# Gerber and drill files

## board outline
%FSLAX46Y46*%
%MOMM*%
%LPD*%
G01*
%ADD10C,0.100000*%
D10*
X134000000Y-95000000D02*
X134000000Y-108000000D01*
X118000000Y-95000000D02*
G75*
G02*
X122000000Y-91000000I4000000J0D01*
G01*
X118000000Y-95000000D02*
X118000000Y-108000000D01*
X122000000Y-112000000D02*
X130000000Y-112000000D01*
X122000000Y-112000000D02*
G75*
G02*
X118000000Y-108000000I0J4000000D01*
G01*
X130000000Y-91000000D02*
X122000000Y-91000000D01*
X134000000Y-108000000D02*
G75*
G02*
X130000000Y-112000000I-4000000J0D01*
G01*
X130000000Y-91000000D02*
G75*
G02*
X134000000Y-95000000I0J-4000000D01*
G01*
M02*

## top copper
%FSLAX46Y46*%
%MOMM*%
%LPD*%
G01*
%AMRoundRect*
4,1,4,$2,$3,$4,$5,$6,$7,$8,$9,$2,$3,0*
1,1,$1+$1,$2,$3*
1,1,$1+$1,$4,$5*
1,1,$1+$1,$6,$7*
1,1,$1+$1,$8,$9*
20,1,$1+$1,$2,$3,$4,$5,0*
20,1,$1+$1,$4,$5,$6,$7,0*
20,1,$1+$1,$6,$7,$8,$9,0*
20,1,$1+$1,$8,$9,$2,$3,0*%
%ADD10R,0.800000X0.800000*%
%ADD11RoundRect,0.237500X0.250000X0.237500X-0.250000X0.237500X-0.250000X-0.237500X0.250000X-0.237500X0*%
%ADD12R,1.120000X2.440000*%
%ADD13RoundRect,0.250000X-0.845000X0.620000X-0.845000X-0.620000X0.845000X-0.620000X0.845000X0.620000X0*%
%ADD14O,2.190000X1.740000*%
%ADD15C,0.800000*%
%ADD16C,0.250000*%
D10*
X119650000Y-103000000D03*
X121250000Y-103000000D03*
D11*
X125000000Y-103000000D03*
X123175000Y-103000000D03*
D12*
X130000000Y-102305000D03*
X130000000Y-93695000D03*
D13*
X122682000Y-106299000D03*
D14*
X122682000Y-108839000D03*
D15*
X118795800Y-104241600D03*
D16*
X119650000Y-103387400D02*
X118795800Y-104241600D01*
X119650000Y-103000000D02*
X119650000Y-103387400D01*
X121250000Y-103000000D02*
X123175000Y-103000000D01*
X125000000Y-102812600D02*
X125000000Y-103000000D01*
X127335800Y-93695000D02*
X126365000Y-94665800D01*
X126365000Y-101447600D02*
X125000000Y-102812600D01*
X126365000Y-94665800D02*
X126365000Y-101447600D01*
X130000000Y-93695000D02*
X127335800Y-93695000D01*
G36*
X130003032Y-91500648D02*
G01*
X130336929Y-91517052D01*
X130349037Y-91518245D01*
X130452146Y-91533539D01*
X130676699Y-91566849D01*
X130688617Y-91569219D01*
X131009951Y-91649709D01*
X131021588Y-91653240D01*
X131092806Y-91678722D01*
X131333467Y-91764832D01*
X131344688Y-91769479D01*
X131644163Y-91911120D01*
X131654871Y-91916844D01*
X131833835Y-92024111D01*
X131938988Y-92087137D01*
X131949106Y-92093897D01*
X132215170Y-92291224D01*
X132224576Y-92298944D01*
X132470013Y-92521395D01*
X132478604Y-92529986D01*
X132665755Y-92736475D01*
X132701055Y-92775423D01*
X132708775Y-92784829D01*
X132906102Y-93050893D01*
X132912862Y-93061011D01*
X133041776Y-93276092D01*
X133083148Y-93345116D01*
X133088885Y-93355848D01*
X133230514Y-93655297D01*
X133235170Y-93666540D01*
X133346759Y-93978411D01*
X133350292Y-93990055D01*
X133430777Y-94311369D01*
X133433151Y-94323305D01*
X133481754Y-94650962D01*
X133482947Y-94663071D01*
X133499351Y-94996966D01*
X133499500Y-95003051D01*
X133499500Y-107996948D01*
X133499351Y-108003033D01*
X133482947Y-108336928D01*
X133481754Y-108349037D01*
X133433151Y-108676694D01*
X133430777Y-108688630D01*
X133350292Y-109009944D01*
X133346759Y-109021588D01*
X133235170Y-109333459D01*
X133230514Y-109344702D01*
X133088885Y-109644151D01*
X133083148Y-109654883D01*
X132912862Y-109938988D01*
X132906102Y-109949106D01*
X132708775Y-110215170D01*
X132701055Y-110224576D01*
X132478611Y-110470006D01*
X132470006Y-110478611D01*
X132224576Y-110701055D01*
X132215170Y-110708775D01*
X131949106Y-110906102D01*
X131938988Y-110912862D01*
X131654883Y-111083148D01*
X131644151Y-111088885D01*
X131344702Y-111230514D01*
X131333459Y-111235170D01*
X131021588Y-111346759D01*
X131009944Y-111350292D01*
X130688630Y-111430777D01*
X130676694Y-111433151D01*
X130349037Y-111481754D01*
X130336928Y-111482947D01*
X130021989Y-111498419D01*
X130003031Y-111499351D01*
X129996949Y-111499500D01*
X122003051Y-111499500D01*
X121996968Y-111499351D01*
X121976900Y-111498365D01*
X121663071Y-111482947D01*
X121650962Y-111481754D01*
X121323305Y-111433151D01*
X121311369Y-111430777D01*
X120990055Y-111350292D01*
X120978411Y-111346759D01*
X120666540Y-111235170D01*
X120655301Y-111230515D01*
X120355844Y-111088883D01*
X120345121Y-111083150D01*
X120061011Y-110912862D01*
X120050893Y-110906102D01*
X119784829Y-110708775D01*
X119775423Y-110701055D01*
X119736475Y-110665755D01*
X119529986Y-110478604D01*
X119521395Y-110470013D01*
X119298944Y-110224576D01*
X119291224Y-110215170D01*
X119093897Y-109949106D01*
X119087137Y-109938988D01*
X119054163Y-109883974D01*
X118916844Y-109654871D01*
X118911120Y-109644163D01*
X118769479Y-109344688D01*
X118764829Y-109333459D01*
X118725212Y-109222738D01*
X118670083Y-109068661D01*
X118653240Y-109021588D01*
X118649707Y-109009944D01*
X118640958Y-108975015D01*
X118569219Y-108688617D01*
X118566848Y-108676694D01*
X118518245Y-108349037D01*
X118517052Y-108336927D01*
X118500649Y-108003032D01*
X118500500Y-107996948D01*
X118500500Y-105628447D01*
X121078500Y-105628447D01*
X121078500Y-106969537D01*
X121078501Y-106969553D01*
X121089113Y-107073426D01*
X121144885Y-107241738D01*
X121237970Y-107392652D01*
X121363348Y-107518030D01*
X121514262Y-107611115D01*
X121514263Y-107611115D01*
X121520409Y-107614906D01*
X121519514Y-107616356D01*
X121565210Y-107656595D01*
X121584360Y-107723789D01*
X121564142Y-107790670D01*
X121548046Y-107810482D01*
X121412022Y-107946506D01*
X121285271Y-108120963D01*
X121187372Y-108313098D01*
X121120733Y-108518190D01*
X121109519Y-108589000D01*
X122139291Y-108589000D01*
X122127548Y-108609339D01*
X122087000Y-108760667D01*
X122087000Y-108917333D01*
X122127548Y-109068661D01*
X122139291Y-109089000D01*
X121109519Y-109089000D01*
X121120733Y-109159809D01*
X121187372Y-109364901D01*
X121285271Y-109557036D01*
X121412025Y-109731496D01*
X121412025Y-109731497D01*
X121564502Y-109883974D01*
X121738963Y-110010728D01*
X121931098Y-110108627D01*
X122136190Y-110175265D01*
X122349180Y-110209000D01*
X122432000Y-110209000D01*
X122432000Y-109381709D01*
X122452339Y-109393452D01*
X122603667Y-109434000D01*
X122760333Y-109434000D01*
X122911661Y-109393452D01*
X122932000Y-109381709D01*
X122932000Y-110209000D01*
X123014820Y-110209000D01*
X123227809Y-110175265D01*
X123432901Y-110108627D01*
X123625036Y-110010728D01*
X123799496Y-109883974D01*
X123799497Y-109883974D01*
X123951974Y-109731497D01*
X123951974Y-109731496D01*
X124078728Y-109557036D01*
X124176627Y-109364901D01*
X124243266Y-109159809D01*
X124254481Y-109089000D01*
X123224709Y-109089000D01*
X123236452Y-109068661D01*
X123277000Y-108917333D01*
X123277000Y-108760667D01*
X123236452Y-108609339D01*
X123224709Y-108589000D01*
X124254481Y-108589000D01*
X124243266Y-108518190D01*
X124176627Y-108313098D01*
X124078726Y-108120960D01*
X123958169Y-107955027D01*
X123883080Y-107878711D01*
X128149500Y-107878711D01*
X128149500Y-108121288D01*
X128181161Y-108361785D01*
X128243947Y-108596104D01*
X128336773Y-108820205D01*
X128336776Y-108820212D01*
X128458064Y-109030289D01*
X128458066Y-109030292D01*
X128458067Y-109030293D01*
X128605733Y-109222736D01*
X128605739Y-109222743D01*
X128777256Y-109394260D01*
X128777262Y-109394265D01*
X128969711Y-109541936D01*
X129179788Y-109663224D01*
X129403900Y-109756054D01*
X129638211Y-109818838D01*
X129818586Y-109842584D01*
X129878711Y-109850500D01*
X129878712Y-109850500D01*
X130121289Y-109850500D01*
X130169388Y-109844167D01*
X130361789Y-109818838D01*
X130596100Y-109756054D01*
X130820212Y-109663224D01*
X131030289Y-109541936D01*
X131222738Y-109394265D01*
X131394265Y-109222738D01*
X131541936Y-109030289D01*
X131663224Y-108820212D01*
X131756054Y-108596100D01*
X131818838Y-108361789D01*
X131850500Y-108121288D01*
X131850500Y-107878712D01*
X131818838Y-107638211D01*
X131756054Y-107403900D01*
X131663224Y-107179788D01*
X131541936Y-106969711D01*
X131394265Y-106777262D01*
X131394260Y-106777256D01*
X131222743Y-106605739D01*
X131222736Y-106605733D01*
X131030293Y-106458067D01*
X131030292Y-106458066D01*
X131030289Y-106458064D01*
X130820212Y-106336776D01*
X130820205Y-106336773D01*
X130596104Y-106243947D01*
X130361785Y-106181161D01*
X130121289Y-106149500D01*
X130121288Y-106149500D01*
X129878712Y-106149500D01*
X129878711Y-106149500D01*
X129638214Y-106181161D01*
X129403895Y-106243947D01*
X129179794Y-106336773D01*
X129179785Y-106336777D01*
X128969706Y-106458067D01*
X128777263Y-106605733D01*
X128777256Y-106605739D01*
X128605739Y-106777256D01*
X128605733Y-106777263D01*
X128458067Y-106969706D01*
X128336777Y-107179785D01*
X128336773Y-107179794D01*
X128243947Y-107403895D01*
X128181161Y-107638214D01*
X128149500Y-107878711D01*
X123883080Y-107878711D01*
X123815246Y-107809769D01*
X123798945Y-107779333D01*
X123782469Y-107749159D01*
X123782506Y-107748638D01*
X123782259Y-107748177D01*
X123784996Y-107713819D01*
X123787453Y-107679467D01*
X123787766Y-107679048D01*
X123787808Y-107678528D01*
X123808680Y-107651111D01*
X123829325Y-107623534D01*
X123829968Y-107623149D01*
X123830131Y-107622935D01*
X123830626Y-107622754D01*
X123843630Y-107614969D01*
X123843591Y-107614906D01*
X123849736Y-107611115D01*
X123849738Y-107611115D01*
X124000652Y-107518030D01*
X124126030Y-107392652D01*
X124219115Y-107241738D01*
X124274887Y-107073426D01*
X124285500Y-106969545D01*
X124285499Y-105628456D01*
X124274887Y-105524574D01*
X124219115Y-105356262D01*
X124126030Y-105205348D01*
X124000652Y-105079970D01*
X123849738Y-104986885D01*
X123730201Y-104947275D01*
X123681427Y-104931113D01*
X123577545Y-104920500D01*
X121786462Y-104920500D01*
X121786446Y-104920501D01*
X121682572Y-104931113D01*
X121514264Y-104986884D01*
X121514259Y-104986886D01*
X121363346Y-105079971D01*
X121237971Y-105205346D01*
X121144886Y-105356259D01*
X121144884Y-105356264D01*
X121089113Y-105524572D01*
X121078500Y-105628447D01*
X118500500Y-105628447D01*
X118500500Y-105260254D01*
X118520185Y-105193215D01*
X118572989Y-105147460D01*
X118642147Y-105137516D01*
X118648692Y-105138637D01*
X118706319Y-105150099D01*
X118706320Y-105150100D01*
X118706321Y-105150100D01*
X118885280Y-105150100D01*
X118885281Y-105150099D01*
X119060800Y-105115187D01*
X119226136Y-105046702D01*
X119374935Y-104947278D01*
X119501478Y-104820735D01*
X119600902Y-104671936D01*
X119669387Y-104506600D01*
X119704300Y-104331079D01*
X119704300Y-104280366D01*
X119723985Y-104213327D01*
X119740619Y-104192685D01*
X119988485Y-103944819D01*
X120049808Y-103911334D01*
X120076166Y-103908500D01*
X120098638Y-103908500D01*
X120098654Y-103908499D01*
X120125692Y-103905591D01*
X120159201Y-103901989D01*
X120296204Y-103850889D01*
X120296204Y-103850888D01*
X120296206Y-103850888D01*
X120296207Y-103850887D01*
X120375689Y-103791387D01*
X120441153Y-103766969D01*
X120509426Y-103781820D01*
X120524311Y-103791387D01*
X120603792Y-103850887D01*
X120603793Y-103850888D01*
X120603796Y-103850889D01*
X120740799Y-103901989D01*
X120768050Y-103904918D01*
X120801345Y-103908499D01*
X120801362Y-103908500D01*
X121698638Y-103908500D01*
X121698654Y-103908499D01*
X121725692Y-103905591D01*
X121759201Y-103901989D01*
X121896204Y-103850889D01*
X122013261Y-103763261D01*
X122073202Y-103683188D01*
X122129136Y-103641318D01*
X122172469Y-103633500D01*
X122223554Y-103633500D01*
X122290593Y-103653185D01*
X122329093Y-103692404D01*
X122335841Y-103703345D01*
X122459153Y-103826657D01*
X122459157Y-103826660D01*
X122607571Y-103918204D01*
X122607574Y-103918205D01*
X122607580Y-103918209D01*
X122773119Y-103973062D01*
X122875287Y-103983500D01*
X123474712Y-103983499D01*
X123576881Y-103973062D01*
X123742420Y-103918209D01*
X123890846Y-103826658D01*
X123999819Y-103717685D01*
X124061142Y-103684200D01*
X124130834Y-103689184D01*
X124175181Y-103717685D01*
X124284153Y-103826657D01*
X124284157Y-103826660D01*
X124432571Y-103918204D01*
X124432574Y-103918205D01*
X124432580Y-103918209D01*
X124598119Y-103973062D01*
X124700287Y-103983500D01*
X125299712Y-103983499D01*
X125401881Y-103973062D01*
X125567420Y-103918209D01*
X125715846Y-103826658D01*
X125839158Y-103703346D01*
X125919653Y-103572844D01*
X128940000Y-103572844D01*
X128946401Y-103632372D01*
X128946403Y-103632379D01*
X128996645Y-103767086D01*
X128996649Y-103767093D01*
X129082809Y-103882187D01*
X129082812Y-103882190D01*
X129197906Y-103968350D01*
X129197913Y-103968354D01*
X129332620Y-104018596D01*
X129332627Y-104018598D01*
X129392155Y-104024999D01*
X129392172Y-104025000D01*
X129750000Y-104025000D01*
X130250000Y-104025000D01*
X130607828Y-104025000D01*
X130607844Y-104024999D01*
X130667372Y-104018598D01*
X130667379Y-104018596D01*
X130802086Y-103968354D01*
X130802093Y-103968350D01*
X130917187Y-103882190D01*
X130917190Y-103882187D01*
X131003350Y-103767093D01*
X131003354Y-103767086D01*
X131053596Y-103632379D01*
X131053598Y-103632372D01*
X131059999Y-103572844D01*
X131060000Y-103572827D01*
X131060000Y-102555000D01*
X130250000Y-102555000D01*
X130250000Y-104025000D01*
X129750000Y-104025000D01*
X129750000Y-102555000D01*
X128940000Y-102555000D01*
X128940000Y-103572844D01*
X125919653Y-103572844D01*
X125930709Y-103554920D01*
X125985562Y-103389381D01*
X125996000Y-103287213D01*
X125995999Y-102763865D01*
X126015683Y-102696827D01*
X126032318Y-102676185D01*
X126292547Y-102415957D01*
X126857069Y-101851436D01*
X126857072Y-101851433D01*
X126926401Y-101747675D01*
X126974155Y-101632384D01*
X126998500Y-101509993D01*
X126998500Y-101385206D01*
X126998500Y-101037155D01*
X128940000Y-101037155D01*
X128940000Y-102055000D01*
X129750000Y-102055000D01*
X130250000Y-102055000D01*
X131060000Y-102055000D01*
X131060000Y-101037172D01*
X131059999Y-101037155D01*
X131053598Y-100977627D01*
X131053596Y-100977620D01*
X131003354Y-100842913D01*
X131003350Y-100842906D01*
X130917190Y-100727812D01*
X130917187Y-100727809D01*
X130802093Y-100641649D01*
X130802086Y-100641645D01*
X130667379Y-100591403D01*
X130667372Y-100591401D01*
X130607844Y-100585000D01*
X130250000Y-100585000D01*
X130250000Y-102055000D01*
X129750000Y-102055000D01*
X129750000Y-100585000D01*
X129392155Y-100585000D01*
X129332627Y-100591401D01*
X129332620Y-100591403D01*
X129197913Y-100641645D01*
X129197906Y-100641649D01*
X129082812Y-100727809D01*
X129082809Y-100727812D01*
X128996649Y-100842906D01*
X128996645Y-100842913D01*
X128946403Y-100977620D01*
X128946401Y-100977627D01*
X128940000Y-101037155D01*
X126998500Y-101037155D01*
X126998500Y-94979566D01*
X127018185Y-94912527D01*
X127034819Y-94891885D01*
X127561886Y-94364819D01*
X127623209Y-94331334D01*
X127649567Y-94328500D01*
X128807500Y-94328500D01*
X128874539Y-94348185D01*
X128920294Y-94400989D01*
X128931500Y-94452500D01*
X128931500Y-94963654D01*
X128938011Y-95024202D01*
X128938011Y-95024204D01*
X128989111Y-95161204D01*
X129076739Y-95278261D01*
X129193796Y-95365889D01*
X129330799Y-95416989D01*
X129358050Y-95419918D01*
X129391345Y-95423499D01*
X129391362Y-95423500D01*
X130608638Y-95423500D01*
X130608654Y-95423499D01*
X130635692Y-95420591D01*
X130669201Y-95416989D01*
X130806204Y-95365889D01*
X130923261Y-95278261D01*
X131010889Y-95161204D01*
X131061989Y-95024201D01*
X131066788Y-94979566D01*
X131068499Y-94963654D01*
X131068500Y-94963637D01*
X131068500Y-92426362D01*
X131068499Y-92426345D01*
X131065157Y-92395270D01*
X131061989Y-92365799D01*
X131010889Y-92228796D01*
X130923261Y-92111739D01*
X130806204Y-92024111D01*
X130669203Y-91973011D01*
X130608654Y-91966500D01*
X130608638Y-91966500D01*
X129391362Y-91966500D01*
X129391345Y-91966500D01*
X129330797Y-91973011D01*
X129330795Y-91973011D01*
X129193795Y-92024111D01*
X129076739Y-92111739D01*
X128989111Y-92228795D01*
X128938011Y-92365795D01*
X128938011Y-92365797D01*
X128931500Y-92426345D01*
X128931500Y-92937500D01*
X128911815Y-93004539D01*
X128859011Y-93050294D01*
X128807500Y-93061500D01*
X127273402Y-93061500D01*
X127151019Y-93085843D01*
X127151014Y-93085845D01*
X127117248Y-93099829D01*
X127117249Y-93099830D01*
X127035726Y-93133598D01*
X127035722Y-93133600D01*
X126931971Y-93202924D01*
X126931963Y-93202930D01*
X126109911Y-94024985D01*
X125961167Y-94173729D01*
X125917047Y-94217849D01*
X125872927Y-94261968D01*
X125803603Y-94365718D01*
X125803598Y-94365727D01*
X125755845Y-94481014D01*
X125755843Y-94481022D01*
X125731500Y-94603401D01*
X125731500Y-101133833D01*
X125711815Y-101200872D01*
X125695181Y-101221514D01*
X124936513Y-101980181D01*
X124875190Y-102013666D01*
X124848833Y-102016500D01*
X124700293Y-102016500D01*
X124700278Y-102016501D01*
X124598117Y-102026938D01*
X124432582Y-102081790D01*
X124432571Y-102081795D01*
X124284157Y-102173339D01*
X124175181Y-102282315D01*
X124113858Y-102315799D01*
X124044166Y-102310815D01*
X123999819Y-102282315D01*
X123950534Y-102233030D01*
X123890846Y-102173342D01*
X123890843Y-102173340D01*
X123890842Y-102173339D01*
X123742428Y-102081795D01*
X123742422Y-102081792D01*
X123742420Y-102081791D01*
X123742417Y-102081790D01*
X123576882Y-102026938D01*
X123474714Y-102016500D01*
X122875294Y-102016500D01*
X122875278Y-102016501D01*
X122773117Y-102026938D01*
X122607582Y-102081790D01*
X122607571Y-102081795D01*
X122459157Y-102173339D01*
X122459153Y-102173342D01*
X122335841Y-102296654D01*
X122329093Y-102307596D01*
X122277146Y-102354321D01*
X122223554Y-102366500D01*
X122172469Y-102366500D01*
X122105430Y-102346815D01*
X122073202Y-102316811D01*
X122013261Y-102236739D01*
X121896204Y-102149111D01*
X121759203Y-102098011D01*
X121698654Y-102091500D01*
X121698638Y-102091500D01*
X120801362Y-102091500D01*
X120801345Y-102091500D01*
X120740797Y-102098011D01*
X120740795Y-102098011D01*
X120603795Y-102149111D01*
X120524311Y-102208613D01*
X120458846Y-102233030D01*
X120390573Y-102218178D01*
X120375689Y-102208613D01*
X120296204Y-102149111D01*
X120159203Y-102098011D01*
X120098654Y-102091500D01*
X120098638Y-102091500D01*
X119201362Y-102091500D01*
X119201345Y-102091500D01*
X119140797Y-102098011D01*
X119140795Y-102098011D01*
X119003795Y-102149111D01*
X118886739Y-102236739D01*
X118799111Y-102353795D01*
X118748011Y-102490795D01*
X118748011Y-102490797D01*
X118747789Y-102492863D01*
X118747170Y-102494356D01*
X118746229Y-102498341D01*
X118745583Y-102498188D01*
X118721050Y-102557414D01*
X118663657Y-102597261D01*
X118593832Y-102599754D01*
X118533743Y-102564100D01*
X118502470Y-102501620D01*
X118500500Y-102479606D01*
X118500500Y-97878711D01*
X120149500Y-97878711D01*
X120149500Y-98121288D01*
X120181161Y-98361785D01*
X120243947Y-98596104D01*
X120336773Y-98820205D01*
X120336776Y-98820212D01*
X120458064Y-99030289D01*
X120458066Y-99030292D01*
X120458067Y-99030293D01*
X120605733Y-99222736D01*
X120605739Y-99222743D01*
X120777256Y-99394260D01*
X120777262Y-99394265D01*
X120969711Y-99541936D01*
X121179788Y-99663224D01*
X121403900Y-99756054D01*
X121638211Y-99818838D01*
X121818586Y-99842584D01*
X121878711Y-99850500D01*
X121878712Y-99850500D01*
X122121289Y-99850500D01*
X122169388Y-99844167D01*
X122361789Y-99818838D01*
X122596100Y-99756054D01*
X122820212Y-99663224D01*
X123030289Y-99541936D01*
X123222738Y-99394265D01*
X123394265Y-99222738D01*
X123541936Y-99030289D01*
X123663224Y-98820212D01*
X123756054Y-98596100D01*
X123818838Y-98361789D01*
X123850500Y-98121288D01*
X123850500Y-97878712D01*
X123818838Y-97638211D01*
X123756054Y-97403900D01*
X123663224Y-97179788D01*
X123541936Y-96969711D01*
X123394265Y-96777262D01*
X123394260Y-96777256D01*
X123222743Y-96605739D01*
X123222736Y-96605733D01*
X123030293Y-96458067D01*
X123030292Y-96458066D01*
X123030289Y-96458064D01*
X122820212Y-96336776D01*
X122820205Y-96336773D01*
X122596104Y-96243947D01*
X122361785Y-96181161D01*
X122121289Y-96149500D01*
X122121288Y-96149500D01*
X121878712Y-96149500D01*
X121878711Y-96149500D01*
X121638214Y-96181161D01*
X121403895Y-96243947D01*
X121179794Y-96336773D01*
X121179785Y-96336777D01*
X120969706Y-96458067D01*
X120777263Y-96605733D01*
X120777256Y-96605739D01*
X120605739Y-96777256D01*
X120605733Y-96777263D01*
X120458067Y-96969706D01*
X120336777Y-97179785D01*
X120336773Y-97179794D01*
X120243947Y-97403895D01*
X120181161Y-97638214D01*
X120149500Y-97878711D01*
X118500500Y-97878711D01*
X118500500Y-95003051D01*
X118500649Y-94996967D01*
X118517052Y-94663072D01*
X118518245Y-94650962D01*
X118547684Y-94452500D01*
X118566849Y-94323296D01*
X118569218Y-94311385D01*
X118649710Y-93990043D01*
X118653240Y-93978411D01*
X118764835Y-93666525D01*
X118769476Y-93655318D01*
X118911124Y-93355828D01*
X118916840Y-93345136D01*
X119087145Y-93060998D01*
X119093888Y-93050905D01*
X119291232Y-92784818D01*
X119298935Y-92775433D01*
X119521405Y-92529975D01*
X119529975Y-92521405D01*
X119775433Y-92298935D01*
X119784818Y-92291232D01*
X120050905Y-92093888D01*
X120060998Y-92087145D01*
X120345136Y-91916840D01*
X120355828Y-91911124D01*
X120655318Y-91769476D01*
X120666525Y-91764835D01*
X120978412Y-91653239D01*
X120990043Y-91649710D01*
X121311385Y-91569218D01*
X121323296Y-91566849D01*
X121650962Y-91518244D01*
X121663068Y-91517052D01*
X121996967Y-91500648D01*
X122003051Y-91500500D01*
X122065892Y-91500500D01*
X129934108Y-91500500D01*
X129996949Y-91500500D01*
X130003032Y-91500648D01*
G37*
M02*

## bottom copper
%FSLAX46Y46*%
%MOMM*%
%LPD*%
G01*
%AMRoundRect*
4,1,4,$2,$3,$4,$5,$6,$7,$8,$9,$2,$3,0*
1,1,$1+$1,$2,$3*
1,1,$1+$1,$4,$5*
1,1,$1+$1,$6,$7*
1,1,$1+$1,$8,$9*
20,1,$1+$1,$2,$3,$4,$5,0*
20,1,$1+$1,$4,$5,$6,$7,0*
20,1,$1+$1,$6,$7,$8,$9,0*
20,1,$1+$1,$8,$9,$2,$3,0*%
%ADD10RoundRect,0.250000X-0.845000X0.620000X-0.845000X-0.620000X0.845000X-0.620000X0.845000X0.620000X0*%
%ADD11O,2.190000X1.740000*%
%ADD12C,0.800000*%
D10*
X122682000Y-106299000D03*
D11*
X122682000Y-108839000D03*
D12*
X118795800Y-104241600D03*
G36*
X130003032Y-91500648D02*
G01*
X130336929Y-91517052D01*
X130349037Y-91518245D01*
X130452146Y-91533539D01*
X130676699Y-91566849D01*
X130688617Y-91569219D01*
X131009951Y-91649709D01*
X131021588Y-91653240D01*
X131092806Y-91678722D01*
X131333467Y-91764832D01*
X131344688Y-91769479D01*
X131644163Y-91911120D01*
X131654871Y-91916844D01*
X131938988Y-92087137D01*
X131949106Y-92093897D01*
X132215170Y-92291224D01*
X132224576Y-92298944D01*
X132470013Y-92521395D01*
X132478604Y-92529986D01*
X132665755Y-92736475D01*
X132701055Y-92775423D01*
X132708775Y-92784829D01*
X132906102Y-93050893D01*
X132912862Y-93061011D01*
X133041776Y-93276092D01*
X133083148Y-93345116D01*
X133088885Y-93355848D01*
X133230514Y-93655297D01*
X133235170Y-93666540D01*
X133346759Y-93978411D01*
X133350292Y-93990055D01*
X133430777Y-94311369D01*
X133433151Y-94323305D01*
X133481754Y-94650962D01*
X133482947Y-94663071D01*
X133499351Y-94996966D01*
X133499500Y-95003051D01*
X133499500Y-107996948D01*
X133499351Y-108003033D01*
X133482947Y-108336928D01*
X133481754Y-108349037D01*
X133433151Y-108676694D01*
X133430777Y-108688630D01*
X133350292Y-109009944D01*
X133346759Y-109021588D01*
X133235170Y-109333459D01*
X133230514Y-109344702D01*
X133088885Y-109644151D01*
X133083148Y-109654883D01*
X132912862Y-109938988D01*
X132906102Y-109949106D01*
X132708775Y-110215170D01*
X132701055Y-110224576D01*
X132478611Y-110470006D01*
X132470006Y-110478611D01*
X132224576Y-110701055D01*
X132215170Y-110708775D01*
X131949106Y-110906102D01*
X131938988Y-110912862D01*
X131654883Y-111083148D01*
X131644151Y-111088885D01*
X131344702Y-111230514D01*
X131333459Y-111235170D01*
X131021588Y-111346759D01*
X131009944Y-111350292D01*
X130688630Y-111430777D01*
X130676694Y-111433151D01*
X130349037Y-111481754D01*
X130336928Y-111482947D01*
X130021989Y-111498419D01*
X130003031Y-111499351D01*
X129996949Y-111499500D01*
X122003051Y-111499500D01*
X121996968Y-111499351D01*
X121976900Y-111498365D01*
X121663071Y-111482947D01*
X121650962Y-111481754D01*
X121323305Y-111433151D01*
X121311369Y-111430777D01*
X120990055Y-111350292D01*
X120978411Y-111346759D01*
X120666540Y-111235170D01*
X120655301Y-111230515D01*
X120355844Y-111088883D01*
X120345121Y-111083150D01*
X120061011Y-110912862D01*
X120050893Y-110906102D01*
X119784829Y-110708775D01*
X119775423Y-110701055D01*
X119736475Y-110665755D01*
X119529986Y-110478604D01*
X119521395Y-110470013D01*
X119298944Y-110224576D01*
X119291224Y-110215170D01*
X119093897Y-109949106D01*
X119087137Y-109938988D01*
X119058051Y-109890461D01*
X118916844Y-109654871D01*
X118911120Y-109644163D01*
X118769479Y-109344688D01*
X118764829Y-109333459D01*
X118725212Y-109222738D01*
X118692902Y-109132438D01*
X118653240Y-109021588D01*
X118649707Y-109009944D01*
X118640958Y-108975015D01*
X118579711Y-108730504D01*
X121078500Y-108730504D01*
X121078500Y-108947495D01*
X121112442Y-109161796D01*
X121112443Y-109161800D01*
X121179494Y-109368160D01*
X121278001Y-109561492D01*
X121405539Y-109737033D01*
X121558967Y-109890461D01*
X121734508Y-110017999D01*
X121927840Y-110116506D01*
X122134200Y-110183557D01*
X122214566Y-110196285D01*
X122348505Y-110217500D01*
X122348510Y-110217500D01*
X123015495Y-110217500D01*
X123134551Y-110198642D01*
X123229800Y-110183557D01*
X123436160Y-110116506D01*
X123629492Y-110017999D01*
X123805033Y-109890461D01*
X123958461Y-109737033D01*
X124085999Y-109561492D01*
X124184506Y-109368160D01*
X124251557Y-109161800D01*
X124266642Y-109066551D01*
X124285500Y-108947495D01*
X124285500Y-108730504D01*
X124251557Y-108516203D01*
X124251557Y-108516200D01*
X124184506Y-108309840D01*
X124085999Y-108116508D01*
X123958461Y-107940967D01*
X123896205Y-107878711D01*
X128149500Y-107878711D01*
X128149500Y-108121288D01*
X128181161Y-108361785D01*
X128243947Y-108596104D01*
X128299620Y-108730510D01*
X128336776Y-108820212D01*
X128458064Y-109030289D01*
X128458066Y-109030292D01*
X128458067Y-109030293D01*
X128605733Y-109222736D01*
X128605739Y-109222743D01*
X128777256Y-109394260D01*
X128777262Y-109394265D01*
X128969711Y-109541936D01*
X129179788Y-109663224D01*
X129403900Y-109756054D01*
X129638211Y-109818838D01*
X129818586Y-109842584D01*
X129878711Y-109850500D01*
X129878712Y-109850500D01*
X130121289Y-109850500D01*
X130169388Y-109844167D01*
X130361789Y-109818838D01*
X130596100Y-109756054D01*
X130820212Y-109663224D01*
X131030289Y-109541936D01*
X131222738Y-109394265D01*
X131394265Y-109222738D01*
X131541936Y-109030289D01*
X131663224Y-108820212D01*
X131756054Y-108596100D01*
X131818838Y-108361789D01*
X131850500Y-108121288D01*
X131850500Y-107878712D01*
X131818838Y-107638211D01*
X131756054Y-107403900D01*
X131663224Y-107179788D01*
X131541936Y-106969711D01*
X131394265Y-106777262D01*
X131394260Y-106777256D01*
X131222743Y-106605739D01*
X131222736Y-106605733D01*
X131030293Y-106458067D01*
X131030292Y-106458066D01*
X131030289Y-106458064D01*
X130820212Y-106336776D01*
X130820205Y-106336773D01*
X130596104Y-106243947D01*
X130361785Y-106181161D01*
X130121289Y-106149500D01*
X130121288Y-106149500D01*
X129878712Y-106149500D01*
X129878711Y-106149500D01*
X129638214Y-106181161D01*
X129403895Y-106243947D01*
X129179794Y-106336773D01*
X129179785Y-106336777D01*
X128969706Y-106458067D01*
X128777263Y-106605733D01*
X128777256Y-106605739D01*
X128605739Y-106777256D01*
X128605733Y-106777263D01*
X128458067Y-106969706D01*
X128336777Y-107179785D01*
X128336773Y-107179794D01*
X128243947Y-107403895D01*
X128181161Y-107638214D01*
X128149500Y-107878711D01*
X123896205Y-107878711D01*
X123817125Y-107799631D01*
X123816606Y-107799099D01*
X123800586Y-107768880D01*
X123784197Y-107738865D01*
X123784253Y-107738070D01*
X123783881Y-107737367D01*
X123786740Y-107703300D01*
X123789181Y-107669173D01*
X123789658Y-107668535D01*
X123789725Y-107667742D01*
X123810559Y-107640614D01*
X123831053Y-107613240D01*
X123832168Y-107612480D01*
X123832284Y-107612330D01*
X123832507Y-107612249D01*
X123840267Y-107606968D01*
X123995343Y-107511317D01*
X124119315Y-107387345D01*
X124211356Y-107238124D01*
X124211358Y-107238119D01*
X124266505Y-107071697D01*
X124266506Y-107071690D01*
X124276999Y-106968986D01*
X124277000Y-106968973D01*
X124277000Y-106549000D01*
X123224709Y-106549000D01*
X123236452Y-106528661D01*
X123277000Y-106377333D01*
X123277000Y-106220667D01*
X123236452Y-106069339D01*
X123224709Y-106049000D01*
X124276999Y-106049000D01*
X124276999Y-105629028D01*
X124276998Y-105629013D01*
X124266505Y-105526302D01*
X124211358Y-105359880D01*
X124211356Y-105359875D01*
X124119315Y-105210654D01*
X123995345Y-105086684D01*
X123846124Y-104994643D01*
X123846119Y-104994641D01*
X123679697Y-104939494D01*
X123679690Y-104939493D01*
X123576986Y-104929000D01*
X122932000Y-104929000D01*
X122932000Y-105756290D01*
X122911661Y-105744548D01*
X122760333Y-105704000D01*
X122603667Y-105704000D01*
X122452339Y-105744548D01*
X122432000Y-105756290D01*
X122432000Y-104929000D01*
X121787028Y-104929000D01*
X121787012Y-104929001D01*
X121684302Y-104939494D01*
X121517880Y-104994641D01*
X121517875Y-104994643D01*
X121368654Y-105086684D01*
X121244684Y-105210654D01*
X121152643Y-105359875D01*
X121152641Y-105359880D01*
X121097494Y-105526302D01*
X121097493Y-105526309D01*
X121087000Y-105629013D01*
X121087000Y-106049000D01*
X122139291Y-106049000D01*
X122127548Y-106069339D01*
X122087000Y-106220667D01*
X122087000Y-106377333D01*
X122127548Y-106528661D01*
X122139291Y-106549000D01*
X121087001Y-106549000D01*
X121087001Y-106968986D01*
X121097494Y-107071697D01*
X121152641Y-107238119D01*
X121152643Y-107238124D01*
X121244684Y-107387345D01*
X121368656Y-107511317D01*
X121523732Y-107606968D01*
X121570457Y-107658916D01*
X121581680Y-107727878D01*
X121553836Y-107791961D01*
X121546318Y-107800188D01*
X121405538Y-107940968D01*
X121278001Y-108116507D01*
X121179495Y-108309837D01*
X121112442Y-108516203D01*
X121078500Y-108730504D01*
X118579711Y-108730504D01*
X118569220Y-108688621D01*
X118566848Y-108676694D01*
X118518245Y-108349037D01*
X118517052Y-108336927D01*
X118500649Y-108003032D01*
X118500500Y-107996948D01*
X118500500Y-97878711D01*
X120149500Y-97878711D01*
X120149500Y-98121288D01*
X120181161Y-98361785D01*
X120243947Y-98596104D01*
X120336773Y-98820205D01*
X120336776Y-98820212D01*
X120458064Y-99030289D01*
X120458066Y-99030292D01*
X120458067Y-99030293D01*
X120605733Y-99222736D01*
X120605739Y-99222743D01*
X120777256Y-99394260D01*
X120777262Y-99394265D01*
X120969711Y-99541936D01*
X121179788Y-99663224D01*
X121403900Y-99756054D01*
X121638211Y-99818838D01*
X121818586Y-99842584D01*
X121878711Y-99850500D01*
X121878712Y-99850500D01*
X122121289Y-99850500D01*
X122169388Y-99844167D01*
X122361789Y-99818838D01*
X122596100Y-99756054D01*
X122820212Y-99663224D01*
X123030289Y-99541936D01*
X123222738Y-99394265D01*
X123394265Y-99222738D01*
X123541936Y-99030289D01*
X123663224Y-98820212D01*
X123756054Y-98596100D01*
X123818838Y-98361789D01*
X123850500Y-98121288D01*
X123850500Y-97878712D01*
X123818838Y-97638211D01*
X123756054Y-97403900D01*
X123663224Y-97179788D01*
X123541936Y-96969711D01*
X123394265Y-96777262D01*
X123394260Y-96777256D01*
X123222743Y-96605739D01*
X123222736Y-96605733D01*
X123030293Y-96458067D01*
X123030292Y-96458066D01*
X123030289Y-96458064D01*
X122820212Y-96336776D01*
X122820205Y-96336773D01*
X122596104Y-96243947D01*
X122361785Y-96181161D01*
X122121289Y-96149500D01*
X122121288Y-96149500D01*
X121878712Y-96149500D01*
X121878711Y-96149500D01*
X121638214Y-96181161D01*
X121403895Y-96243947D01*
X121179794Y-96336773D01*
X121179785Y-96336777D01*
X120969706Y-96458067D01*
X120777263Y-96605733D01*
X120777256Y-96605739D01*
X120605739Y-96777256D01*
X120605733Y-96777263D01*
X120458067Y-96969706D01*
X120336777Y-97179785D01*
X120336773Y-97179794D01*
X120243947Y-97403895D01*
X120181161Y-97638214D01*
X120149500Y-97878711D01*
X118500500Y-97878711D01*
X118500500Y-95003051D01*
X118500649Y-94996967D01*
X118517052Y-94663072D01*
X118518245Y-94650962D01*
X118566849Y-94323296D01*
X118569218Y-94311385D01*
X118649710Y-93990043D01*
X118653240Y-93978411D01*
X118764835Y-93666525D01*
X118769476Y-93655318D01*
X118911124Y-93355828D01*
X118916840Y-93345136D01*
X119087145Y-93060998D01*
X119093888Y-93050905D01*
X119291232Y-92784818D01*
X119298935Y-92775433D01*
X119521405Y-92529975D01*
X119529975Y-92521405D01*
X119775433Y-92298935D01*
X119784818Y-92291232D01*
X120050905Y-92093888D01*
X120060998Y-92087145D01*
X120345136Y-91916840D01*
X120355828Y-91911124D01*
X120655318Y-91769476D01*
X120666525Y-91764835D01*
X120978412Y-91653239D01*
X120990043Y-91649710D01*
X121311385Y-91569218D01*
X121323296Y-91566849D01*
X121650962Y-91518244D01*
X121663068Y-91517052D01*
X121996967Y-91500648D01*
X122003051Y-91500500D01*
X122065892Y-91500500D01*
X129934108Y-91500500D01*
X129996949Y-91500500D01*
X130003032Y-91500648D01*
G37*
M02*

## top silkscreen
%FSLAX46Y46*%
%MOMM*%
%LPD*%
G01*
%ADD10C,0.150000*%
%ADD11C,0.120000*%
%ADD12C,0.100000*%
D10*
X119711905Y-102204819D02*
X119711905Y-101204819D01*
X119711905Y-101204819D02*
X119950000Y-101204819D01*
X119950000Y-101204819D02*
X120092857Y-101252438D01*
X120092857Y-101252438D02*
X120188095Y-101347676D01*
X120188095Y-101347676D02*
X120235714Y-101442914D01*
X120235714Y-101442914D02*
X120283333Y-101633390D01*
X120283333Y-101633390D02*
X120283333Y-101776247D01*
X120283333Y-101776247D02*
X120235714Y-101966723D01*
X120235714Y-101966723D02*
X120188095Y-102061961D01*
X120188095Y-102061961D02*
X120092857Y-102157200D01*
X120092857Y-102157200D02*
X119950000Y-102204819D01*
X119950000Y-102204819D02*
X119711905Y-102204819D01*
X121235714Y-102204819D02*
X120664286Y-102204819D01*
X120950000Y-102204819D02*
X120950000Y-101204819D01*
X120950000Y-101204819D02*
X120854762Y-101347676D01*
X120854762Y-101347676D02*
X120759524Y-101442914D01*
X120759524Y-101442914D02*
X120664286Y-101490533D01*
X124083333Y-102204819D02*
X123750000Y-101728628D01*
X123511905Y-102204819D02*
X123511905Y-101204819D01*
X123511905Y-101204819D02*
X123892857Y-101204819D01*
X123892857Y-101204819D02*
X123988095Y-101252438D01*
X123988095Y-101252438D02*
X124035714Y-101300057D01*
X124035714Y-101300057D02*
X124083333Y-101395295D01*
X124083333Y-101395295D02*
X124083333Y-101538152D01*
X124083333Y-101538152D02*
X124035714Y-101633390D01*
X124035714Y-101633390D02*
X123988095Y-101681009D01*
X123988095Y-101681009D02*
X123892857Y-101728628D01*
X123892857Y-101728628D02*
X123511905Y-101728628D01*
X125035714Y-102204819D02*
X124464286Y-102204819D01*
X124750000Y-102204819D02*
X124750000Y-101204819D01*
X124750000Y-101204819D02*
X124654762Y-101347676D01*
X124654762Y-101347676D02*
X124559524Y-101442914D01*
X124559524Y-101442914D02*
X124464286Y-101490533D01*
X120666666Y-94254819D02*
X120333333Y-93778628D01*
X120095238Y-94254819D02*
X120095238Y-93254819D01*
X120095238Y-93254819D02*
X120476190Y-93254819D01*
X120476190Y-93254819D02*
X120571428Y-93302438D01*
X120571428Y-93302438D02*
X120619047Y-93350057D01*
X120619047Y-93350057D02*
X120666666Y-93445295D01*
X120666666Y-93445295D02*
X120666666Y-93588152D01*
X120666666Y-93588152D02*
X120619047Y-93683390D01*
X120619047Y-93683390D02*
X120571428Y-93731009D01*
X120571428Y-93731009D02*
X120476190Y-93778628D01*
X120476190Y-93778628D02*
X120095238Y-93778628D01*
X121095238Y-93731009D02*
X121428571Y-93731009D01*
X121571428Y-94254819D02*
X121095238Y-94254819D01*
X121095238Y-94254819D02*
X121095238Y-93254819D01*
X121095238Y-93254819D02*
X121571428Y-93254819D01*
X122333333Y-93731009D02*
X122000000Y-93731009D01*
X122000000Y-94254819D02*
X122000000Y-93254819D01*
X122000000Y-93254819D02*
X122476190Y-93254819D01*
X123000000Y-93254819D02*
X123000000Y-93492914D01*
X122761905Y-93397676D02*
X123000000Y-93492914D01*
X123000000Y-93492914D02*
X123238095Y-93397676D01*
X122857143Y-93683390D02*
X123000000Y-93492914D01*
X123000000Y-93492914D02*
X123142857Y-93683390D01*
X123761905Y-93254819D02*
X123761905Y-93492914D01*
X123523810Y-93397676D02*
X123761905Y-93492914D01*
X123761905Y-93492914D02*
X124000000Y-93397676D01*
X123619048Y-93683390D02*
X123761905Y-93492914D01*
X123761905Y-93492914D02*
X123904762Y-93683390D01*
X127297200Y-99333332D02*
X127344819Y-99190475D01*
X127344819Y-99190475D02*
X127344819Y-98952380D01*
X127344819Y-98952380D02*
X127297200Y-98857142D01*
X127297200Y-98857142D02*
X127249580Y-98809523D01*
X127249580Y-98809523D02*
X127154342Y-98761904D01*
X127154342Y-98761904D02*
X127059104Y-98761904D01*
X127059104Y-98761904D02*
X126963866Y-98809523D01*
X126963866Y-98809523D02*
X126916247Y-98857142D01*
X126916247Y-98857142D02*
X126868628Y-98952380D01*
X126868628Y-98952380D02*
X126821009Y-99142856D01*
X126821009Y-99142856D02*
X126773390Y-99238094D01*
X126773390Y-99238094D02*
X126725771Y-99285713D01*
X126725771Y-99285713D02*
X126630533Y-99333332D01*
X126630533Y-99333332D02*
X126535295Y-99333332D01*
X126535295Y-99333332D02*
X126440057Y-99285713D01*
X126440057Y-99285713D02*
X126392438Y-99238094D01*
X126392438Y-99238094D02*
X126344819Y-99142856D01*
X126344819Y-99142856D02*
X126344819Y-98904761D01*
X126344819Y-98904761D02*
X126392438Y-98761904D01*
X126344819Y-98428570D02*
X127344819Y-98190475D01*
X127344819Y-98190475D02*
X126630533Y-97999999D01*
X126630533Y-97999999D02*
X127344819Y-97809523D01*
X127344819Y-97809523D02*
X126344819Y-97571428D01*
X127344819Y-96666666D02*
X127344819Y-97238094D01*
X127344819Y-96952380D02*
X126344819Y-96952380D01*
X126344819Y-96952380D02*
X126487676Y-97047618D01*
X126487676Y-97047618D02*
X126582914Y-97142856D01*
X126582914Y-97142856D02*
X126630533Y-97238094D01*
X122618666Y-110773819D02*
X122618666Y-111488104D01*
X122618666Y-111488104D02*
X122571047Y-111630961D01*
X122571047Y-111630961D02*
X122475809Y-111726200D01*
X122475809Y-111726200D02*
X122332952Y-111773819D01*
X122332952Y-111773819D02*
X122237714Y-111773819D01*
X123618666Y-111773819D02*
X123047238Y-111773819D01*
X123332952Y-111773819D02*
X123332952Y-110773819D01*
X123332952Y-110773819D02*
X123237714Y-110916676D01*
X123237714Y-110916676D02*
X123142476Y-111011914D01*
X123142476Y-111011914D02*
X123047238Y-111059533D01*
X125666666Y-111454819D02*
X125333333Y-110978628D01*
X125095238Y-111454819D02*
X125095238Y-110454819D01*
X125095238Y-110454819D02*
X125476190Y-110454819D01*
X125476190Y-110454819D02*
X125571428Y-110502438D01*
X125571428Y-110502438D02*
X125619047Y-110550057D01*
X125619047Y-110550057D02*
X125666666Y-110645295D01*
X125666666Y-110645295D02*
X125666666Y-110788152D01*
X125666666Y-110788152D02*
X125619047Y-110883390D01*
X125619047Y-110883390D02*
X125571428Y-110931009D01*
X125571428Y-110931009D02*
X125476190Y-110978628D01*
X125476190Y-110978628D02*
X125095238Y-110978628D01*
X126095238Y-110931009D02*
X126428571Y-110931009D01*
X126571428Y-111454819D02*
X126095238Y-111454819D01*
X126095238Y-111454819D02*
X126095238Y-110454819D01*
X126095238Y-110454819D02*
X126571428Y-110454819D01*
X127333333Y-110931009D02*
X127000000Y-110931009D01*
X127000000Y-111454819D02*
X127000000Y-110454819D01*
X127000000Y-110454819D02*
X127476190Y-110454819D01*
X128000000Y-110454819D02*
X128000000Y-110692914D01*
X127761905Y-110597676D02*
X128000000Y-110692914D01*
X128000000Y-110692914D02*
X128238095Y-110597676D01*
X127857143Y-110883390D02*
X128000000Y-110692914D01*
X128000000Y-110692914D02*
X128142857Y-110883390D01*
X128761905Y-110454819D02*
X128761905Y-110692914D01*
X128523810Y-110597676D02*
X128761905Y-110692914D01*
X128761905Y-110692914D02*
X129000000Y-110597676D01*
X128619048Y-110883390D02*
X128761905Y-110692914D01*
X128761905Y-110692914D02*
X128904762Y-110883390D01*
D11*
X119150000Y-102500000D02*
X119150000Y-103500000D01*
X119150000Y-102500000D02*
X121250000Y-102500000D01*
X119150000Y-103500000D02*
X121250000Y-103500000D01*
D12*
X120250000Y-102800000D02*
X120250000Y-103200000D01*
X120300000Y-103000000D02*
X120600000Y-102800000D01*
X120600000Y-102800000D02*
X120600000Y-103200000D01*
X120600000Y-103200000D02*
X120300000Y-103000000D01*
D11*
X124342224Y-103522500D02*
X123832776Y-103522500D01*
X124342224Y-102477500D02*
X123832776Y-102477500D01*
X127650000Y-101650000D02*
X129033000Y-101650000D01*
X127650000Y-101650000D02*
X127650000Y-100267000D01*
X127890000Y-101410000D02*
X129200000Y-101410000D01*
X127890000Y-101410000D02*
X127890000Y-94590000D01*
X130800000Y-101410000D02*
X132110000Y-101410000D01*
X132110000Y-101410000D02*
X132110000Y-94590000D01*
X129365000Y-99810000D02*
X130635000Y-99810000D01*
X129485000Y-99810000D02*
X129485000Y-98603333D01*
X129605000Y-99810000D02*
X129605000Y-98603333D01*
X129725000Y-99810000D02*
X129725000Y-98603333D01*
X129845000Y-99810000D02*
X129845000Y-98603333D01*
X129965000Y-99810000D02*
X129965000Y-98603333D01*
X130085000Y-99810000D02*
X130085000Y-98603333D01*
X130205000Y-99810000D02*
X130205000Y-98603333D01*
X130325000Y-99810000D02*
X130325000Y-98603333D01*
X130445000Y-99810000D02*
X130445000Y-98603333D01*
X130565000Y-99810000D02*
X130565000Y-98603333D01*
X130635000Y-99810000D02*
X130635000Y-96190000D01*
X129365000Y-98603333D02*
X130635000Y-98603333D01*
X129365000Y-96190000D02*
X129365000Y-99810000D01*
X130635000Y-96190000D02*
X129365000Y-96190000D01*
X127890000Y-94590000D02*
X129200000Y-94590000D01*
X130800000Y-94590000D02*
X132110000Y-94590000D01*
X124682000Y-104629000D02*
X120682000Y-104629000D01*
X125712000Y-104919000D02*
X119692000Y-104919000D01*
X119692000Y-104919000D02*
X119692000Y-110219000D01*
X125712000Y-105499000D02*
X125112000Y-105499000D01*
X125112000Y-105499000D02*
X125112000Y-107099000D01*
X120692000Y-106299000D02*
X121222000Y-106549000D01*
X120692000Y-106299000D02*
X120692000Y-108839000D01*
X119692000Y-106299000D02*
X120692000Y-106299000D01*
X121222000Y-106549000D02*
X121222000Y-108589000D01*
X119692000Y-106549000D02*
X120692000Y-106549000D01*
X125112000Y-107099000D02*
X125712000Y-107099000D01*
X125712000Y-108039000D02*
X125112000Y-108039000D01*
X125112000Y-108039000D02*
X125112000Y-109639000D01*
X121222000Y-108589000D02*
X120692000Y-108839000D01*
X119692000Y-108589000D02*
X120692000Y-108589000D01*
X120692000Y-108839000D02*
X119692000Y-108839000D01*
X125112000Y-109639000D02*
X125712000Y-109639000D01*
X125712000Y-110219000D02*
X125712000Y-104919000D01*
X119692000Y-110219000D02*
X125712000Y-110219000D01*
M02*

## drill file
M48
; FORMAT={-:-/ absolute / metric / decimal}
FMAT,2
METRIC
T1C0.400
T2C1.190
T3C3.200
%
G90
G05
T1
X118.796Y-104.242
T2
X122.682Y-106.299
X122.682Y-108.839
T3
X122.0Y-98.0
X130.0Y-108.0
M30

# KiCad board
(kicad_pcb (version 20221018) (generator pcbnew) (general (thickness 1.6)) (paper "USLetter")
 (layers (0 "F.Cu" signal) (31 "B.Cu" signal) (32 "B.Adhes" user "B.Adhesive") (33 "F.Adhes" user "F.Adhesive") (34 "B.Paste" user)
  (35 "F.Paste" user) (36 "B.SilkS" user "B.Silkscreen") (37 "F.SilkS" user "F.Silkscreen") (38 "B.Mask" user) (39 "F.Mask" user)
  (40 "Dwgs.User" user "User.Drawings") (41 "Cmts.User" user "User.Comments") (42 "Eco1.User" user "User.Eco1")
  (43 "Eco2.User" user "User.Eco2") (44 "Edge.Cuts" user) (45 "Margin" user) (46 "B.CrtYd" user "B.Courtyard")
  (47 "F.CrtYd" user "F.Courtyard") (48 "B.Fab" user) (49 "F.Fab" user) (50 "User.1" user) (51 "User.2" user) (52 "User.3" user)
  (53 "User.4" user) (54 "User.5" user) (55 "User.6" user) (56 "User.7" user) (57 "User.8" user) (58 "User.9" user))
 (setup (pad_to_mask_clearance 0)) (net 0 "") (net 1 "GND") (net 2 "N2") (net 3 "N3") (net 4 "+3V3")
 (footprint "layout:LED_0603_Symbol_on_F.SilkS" (layer "F.Cu") (at 120.45 103)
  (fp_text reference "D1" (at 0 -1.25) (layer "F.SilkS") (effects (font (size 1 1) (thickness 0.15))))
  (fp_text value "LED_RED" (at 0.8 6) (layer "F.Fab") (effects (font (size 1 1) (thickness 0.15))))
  (fp_line (start -1.3 -0.5) (end -1.3 0.5) (stroke (width 0.12) (type solid)) (layer "F.SilkS"))
  (fp_line (start -1.3 -0.5) (end 0.8 -0.5) (stroke (width 0.12) (type solid)) (layer "F.SilkS"))
  (fp_line (start -1.3 0.5) (end 0.8 0.5) (stroke (width 0.12) (type solid)) (layer "F.SilkS"))
  (fp_line (start -0.2 -0.2) (end -0.2 0.2) (stroke (width 0.1) (type solid)) (layer "F.SilkS"))
  (fp_line (start -0.15 0) (end 0.15 -0.2) (stroke (width 0.1) (type solid)) (layer "F.SilkS"))
  (fp_line (start 0.15 -0.2) (end 0.15 0.2) (stroke (width 0.1) (type solid)) (layer "F.SilkS"))
  (fp_line (start 0.15 0.2) (end -0.15 0) (stroke (width 0.1) (type solid)) (layer "F.SilkS"))
  (pad "1" smd rect (at -0.8 0 180) (size 0.8 0.8) (layers "F.Cu" "F.Paste" "F.Mask") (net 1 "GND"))
  (pad "2" smd rect (at 0.8 0 180) (size 0.8 0.8) (layers "F.Cu" "F.Paste" "F.Mask") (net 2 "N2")))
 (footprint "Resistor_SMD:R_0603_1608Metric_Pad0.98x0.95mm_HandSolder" (layer "F.Cu") (at 124.0875 103 180)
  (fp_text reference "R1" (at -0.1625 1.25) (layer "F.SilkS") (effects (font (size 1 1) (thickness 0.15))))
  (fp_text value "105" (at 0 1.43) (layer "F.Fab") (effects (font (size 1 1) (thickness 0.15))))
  (fp_line (start -0.254724 -0.5225) (end 0.254724 -0.5225) (stroke (width 0.12) (type solid)) (layer "F.SilkS"))
  (fp_line (start -0.254724 0.5225) (end 0.254724 0.5225) (stroke (width 0.12) (type solid)) (layer "F.SilkS"))
  (pad "1" smd roundrect (at -0.9125 0 180) (size 0.975 0.95) (layers "F.Cu" "F.Paste" "F.Mask") (roundrect_rratio 0.25) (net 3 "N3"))
  (pad "2" smd roundrect (at 0.9125 0 180) (size 0.975 0.95) (layers "F.Cu" "F.Paste" "F.Mask") (roundrect_rratio 0.25) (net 2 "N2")))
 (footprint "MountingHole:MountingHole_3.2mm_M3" (layer "F.Cu") (at 122 98)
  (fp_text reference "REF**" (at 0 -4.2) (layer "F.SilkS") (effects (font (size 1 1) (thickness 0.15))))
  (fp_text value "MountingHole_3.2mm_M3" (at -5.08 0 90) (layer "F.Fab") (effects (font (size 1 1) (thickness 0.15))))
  (pad "" np_thru_hole circle (at 0 0) (size 3.2 3.2) (drill 3.2) (layers "*.Cu" "*.Mask")))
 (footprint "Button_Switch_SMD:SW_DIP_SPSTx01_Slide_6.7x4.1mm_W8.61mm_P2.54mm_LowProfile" (layer "F.Cu") (at 130 98 90)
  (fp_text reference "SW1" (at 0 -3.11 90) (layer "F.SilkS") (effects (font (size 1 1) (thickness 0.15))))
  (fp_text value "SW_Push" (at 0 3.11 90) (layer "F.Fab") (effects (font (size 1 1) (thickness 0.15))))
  (fp_line (start -3.65 -2.35) (end -3.65 -0.967) (stroke (width 0.12) (type solid)) (layer "F.SilkS"))
  (fp_line (start -3.65 -2.35) (end -2.267 -2.35) (stroke (width 0.12) (type solid)) (layer "F.SilkS"))
  (fp_line (start -3.41 -2.11) (end -3.41 -0.8) (stroke (width 0.12) (type solid)) (layer "F.SilkS"))
  (fp_line (start -3.41 -2.11) (end 3.41 -2.11) (stroke (width 0.12) (type solid)) (layer "F.SilkS"))
  (fp_line (start -3.41 0.8) (end -3.41 2.11) (stroke (width 0.12) (type solid)) (layer "F.SilkS"))
  (fp_line (start -3.41 2.11) (end 3.41 2.11) (stroke (width 0.12) (type solid)) (layer "F.SilkS"))
  (fp_line (start -1.81 -0.635) (end -1.81 0.635) (stroke (width 0.12) (type solid)) (layer "F.SilkS"))
  (fp_line (start -1.81 -0.515) (end -0.603333 -0.515) (stroke (width 0.12) (type solid)) (layer "F.SilkS"))
  (fp_line (start -1.81 -0.395) (end -0.603333 -0.395) (stroke (width 0.12) (type solid)) (layer "F.SilkS"))
  (fp_line (start -1.81 -0.275) (end -0.603333 -0.275) (stroke (width 0.12) (type solid)) (layer "F.SilkS"))
  (fp_line (start -1.81 -0.155) (end -0.603333 -0.155) (stroke (width 0.12) (type solid)) (layer "F.SilkS"))
  (fp_line (start -1.81 -0.035) (end -0.603333 -0.035) (stroke (width 0.12) (type solid)) (layer "F.SilkS"))
  (fp_line (start -1.81 0.085) (end -0.603333 0.085) (stroke (width 0.12) (type solid)) (layer "F.SilkS"))
  (fp_line (start -1.81 0.205) (end -0.603333 0.205) (stroke (width 0.12) (type solid)) (layer "F.SilkS"))
  (fp_line (start -1.81 0.325) (end -0.603333 0.325) (stroke (width 0.12) (type solid)) (layer "F.SilkS"))
  (fp_line (start -1.81 0.445) (end -0.603333 0.445) (stroke (width 0.12) (type solid)) (layer "F.SilkS"))
  (fp_line (start -1.81 0.565) (end -0.603333 0.565) (stroke (width 0.12) (type solid)) (layer "F.SilkS"))
  (fp_line (start -1.81 0.635) (end 1.81 0.635) (stroke (width 0.12) (type solid)) (layer "F.SilkS"))
  (fp_line (start -0.603333 -0.635) (end -0.603333 0.635) (stroke (width 0.12) (type solid)) (layer "F.SilkS"))
  (fp_line (start 1.81 -0.635) (end -1.81 -0.635) (stroke (width 0.12) (type solid)) (layer "F.SilkS"))
  (fp_line (start 1.81 0.635) (end 1.81 -0.635) (stroke (width 0.12) (type solid)) (layer "F.SilkS"))
  (fp_line (start 3.41 -2.11) (end 3.41 -0.8) (stroke (width 0.12) (type solid)) (layer "F.SilkS"))
  (fp_line (start 3.41 0.8) (end 3.41 2.11) (stroke (width 0.12) (type solid)) (layer "F.SilkS"))
  (pad "1" smd rect (at -4.305 0 90) (size 2.44 1.12) (layers "F.Cu" "F.Paste" "F.Mask") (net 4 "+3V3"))
  (pad "2" smd rect (at 4.305 0 90) (size 2.44 1.12) (layers "F.Cu" "F.Paste" "F.Mask") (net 3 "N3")))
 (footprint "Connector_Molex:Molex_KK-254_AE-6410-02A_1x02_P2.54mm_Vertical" (layer "F.Cu") (at 122.682 106.299 -90)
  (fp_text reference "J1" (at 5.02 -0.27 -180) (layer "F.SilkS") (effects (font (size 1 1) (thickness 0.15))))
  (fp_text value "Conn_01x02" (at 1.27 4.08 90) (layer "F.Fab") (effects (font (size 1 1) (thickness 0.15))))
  (fp_line (start -1.67 -2) (end -1.67 2) (stroke (width 0.12) (type solid)) (layer "F.SilkS"))
  (fp_line (start -1.38 -3.03) (end -1.38 2.99) (stroke (width 0.12) (type solid)) (layer "F.SilkS"))
  (fp_line (start -1.38 2.99) (end 3.92 2.99) (stroke (width 0.12) (type solid)) (layer "F.SilkS"))
  (fp_line (start -0.8 -3.03) (end -0.8 -2.43) (stroke (width 0.12) (type solid)) (layer "F.SilkS"))
  (fp_line (start -0.8 -2.43) (end 0.8 -2.43) (stroke (width 0.12) (type solid)) (layer "F.SilkS"))
  (fp_line (start 0 1.99) (end 0.25 1.46) (stroke (width 0.12) (type solid)) (layer "F.SilkS"))
  (fp_line (start 0 1.99) (end 2.54 1.99) (stroke (width 0.12) (type solid)) (layer "F.SilkS"))
  (fp_line (start 0 2.99) (end 0 1.99) (stroke (width 0.12) (type solid)) (layer "F.SilkS"))
  (fp_line (start 0.25 1.46) (end 2.29 1.46) (stroke (width 0.12) (type solid)) (layer "F.SilkS"))
  (fp_line (start 0.25 2.99) (end 0.25 1.99) (stroke (width 0.12) (type solid)) (layer "F.SilkS"))
  (fp_line (start 0.8 -2.43) (end 0.8 -3.03) (stroke (width 0.12) (type solid)) (layer "F.SilkS"))
  (fp_line (start 1.74 -3.03) (end 1.74 -2.43) (stroke (width 0.12) (type solid)) (layer "F.SilkS"))
  (fp_line (start 1.74 -2.43) (end 3.34 -2.43) (stroke (width 0.12) (type solid)) (layer "F.SilkS"))
  (fp_line (start 2.29 1.46) (end 2.54 1.99) (stroke (width 0.12) (type solid)) (layer "F.SilkS"))
  (fp_line (start 2.29 2.99) (end 2.29 1.99) (stroke (width 0.12) (type solid)) (layer "F.SilkS"))
  (fp_line (start 2.54 1.99) (end 2.54 2.99) (stroke (width 0.12) (type solid)) (layer "F.SilkS"))
  (fp_line (start 3.34 -2.43) (end 3.34 -3.03) (stroke (width 0.12) (type solid)) (layer "F.SilkS"))
  (fp_line (start 3.92 -3.03) (end -1.38 -3.03) (stroke (width 0.12) (type solid)) (layer "F.SilkS"))
  (fp_line (start 3.92 2.99) (end 3.92 -3.03) (stroke (width 0.12) (type solid)) (layer "F.SilkS"))
  (pad "1" thru_hole roundrect (at 0 0 270) (size 1.74 2.19) (drill 1.19) (layers "*.Cu" "*.Mask") (roundrect_rratio 0.1436781609)
   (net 1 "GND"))
  (pad "2" thru_hole oval (at 2.54 0 270) (size 1.74 2.19) (drill 1.19) (layers "*.Cu" "*.Mask") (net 4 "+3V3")))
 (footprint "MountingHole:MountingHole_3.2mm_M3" (layer "F.Cu") (at 130 108)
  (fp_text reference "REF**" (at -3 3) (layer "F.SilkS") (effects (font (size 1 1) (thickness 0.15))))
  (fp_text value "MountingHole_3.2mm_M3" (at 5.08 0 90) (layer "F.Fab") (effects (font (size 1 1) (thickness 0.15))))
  (pad "" np_thru_hole circle (at 0 0) (size 3.2 3.2) (drill 3.2) (layers "F&B.Cu" "*.Mask")))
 (gr_line (start 134 95) (end 134 108) (stroke (width 0.1) (type default)) (layer "Edge.Cuts"))
 (gr_arc (start 118 95) (mid 119.171573 92.171573) (end 122 91) (stroke (width 0.1) (type default)) (layer "Edge.Cuts"))
 (gr_line (start 118 95) (end 118 108) (stroke (width 0.1) (type default)) (layer "Edge.Cuts"))
 (gr_line (start 122 112) (end 130 112) (stroke (width 0.1) (type default)) (layer "Edge.Cuts"))
 (gr_arc (start 122 112) (mid 119.171573 110.828427) (end 118 108) (stroke (width 0.1) (type default)) (layer "Edge.Cuts"))
 (gr_line (start 130 91) (end 122 91) (stroke (width 0.1) (type default)) (layer "Edge.Cuts"))
 (gr_arc (start 134 108) (mid 132.828427 110.828427) (end 130 112) (stroke (width 0.1) (type default)) (layer "Edge.Cuts"))
 (gr_arc (start 130 91) (mid 132.828427 92.171573) (end 134 95) (stroke (width 0.1) (type default)) (layer "Edge.Cuts"))
 (segment (start 119.65 103.3874) (end 118.7958 104.2416) (width 0.25) (layer "F.Cu") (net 1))
 (segment (start 119.65 103) (end 119.65 103.3874) (width 0.25) (layer "F.Cu") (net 1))
 (via (at 118.7958 104.2416) (size 0.8) (drill 0.4) (layers "F.Cu" "B.Cu") (free) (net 1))
 (segment (start 121.25 103) (end 123.175 103) (width 0.25) (layer "F.Cu") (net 2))
 (segment (start 125 102.8126) (end 125 103) (width 0.25) (layer "F.Cu") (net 3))
 (segment (start 127.3358 93.695) (end 126.365 94.6658) (width 0.25) (layer "F.Cu") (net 3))
 (segment (start 126.365 101.4476) (end 125 102.8126) (width 0.25) (layer "F.Cu") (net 3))
 (segment (start 126.365 94.6658) (end 126.365 101.4476) (width 0.25) (layer "F.Cu") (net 3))
 (segment (start 130 93.695) (end 127.3358 93.695) (width 0.25) (layer "F.Cu") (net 3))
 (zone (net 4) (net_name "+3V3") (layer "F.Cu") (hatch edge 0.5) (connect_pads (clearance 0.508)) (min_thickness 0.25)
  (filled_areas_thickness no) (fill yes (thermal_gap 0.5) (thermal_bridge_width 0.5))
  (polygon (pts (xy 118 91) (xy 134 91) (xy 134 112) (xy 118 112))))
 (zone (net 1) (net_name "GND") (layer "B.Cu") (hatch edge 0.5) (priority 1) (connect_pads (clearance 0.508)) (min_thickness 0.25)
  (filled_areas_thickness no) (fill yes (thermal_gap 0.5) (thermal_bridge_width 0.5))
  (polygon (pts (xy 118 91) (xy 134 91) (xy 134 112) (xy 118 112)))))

